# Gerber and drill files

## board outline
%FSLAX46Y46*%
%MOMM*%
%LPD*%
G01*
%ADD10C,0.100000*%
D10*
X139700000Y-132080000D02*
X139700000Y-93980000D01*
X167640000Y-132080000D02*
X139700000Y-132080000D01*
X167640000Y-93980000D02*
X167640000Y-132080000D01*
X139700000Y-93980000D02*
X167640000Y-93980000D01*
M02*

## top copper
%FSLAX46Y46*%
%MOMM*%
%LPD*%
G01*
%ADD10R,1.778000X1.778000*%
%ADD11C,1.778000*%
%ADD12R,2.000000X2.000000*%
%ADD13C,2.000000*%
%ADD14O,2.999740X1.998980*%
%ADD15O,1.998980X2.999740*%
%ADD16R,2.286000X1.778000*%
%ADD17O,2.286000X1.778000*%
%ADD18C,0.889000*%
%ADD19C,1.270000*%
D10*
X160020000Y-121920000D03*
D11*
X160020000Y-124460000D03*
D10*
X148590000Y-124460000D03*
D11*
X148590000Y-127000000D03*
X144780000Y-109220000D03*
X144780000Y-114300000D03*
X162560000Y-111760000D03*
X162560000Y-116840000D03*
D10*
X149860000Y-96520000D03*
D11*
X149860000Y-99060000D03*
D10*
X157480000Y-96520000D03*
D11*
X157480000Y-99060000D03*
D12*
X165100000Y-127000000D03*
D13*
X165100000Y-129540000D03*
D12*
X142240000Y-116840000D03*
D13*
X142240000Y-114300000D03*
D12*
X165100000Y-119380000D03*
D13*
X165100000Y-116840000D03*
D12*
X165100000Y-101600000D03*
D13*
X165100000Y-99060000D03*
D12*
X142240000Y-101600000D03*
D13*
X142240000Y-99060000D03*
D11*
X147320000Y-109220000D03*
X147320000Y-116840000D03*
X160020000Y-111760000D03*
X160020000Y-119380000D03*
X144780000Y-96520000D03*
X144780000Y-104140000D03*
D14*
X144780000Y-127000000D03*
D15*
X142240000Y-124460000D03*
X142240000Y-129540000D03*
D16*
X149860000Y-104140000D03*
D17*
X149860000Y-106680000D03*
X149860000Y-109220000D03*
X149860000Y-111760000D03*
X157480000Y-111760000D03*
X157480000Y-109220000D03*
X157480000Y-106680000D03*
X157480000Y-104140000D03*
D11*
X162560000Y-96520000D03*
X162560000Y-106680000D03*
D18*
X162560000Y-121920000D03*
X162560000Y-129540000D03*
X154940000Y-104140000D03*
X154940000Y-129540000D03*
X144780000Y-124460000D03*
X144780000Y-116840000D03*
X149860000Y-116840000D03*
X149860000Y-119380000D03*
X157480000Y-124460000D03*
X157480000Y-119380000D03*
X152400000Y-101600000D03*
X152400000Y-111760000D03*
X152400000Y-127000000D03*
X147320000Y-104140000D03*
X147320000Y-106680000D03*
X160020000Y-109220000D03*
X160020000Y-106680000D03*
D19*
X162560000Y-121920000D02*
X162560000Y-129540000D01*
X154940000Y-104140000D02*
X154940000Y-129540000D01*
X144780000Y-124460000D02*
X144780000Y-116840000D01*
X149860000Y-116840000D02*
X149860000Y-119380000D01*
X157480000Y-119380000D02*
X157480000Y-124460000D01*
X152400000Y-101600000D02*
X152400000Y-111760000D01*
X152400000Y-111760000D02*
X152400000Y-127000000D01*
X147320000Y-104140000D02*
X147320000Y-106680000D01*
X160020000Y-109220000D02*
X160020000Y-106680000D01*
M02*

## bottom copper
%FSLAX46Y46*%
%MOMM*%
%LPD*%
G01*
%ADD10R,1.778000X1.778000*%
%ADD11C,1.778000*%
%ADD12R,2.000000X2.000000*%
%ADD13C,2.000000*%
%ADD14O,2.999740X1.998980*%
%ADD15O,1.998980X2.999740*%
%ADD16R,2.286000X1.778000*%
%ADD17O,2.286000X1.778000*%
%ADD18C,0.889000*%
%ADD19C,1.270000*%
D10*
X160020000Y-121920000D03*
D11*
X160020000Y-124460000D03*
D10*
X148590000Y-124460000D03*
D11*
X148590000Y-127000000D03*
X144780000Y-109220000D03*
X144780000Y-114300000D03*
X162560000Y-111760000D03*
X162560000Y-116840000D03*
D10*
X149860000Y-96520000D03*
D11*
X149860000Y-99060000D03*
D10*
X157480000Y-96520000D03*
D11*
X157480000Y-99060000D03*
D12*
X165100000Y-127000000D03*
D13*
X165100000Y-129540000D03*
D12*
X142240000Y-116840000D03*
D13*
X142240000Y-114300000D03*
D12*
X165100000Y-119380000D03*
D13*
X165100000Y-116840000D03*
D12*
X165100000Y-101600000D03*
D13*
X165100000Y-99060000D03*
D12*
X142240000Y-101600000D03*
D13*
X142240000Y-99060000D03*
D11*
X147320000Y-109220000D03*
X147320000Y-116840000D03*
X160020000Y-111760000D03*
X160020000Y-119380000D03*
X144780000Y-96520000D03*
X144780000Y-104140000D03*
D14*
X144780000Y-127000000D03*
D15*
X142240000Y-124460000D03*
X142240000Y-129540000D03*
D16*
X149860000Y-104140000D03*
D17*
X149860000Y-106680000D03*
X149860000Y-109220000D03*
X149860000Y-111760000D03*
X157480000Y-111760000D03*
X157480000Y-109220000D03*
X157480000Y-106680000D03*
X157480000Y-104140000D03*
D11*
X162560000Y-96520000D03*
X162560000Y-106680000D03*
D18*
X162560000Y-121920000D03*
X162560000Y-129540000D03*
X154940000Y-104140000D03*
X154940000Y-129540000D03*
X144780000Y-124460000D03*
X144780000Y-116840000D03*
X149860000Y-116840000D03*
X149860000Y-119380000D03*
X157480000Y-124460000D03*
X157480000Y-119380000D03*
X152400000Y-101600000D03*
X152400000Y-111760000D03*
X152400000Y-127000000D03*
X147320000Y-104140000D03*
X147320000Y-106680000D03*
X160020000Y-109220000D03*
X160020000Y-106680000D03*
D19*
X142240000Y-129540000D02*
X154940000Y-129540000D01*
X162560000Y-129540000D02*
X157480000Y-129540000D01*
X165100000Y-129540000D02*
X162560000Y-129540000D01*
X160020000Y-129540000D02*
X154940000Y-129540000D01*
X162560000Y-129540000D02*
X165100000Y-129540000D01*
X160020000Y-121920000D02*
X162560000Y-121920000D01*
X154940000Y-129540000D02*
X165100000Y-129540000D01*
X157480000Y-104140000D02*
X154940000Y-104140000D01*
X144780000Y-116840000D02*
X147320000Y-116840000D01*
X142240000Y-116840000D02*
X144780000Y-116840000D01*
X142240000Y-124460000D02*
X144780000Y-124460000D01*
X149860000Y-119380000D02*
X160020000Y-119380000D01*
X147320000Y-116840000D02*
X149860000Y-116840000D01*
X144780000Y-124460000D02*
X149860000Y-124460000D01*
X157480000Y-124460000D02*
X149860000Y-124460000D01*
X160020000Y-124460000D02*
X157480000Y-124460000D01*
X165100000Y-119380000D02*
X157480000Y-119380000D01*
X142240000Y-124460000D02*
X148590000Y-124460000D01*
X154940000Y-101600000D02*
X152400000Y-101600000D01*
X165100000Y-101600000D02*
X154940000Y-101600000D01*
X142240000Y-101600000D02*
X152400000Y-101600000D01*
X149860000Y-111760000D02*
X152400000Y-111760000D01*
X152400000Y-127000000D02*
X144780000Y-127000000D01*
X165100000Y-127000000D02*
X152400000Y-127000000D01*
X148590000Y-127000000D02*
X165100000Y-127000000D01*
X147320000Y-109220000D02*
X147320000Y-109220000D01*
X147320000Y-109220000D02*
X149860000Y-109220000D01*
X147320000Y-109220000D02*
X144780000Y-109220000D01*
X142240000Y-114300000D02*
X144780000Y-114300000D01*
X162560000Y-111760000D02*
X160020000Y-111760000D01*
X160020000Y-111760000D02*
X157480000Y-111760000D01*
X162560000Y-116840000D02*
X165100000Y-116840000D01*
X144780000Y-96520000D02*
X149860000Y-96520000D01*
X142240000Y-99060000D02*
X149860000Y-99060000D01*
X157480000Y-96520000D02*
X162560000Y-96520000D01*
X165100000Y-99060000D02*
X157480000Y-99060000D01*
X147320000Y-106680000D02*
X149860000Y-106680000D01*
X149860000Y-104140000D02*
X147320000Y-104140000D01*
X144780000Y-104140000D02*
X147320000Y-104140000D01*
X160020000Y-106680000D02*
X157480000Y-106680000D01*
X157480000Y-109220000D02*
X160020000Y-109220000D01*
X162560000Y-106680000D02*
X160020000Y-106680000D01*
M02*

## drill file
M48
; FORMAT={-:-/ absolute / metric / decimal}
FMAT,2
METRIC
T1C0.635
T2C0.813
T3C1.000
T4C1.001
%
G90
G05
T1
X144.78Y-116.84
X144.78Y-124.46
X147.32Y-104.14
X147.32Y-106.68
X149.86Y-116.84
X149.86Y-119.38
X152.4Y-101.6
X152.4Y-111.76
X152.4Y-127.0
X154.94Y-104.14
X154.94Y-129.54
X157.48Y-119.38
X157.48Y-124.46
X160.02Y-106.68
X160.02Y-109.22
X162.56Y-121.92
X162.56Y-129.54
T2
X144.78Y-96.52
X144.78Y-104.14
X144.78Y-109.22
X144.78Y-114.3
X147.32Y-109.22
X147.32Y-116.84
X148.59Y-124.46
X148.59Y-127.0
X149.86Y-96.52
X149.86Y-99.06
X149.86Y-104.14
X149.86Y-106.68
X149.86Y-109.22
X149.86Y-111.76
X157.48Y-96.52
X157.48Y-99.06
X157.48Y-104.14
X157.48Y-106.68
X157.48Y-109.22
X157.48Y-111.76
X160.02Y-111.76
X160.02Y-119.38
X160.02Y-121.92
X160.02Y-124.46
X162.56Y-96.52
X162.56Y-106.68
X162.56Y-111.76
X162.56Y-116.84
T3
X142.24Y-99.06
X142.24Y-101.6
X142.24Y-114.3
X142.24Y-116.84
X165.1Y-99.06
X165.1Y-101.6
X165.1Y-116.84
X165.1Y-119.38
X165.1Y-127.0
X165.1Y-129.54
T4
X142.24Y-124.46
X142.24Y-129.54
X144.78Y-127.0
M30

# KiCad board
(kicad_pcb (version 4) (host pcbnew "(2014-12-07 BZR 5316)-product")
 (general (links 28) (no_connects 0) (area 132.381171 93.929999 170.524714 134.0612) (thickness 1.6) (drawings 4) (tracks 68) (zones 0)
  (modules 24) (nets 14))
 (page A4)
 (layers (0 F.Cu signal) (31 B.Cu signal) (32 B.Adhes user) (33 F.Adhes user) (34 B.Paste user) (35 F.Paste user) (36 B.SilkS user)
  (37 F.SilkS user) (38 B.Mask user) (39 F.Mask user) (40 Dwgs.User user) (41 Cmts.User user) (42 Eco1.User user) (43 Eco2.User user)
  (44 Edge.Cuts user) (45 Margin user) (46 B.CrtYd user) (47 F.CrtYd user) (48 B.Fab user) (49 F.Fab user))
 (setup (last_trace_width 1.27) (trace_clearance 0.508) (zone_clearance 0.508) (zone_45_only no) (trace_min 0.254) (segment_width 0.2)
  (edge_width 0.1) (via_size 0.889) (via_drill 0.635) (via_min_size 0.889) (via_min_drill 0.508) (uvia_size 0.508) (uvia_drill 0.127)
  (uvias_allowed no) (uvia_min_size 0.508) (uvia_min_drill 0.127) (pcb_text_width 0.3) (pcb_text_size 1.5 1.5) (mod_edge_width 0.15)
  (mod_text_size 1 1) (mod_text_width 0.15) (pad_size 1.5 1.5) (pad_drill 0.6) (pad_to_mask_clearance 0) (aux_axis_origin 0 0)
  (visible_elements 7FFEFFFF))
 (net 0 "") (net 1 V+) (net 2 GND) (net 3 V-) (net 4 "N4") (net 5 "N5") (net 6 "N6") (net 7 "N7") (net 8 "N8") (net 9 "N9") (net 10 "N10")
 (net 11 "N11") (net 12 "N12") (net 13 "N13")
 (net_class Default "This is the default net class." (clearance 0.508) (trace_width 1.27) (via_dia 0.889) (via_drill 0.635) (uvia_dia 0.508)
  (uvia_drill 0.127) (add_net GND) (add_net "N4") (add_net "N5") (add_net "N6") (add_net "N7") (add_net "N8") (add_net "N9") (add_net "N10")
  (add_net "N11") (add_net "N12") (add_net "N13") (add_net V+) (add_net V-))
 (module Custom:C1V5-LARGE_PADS (layer F.Cu) (at 160.02 123.19 270)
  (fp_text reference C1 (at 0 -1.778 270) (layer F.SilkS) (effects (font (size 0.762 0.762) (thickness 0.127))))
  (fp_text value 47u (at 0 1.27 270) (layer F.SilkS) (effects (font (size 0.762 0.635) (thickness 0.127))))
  (pad 1 thru_hole rect (at -1.27 0 270) (size 1.778 1.778) (drill 0.8128) (layers *.Cu *.Mask F.SilkS) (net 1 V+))
  (pad 2 thru_hole circle (at 1.27 0 270) (size 1.778 1.778) (drill 0.8128) (layers *.Cu *.Mask F.SilkS) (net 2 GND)))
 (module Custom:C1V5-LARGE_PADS (layer F.Cu) (at 148.59 125.73 270)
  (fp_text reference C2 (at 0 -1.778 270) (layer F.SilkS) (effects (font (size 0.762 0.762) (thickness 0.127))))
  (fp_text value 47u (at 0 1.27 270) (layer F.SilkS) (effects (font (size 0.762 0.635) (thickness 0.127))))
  (pad 1 thru_hole rect (at -1.27 0 270) (size 1.778 1.778) (drill 0.8128) (layers *.Cu *.Mask F.SilkS) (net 2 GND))
  (pad 2 thru_hole circle (at 1.27 0 270) (size 1.778 1.778) (drill 0.8128) (layers *.Cu *.Mask F.SilkS) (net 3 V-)))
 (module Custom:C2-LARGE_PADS (layer F.Cu) (at 144.78 111.76 270)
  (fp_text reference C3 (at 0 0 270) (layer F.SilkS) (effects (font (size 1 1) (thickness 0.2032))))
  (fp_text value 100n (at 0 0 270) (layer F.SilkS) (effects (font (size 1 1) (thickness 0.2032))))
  (pad 1 thru_hole circle (at -2.54 0 270) (size 1.778 1.778) (drill 0.8128) (layers *.Cu *.Mask F.SilkS) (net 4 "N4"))
  (pad 2 thru_hole circle (at 2.54 0 270) (size 1.778 1.778) (drill 0.8128) (layers *.Cu *.Mask F.SilkS) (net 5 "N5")))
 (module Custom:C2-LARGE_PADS (layer F.Cu) (at 162.56 114.3 270)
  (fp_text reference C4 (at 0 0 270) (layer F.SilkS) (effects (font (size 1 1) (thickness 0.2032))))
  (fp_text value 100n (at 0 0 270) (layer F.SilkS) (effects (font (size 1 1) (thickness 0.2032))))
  (pad 1 thru_hole circle (at -2.54 0 270) (size 1.778 1.778) (drill 0.8128) (layers *.Cu *.Mask F.SilkS) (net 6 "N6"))
  (pad 2 thru_hole circle (at 2.54 0 270) (size 1.778 1.778) (drill 0.8128) (layers *.Cu *.Mask F.SilkS) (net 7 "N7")))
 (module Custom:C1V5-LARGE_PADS (layer F.Cu) (at 149.86 97.79 270)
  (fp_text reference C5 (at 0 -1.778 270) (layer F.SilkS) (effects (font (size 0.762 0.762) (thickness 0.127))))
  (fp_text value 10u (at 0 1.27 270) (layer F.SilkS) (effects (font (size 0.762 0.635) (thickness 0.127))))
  (pad 1 thru_hole rect (at -1.27 0 270) (size 1.778 1.778) (drill 0.8128) (layers *.Cu *.Mask F.SilkS) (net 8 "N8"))
  (pad 2 thru_hole circle (at 1.27 0 270) (size 1.778 1.778) (drill 0.8128) (layers *.Cu *.Mask F.SilkS) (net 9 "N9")))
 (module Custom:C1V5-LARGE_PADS (layer F.Cu) (at 157.48 97.79 270)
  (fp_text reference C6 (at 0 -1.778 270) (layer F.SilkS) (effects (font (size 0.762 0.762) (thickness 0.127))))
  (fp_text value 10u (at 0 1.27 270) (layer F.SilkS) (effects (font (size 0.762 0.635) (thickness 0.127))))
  (pad 1 thru_hole rect (at -1.27 0 270) (size 1.778 1.778) (drill 0.8128) (layers *.Cu *.Mask F.SilkS) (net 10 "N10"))
  (pad 2 thru_hole circle (at 1.27 0 270) (size 1.778 1.778) (drill 0.8128) (layers *.Cu *.Mask F.SilkS) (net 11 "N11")))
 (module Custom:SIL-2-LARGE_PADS (layer F.Cu) (at 165.1 128.27 270)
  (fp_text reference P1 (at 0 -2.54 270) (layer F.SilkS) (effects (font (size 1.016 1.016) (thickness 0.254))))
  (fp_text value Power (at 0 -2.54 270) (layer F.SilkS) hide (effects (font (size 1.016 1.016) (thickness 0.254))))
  (pad 1 thru_hole rect (at -1.27 0 270) (size 2 2) (drill 1) (layers *.Cu *.Mask F.SilkS) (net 3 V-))
  (pad 2 thru_hole circle (at 1.27 0 270) (size 2 2) (drill 1) (layers *.Cu *.Mask F.SilkS) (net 1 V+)))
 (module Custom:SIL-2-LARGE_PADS (layer F.Cu) (at 142.24 115.57 90)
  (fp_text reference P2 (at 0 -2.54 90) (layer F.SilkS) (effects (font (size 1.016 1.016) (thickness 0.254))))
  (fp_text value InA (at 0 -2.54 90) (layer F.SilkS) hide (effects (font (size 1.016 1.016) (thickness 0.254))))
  (pad 1 thru_hole rect (at -1.27 0 90) (size 2 2) (drill 1) (layers *.Cu *.Mask F.SilkS) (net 2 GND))
  (pad 2 thru_hole circle (at 1.27 0 90) (size 2 2) (drill 1) (layers *.Cu *.Mask F.SilkS) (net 5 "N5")))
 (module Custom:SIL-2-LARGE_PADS (layer F.Cu) (at 165.1 118.11 90)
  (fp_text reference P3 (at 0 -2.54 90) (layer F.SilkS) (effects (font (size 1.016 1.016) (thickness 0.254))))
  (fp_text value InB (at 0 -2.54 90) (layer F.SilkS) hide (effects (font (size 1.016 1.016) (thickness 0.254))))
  (pad 1 thru_hole rect (at -1.27 0 90) (size 2 2) (drill 1) (layers *.Cu *.Mask F.SilkS) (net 2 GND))
  (pad 2 thru_hole circle (at 1.27 0 90) (size 2 2) (drill 1) (layers *.Cu *.Mask F.SilkS) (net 7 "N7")))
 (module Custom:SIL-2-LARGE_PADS (layer F.Cu) (at 165.1 100.33 90)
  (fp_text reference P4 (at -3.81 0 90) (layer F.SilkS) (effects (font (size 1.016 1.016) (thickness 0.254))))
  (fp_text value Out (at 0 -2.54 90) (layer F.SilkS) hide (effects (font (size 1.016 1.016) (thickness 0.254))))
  (pad 1 thru_hole rect (at -1.27 0 90) (size 2 2) (drill 1) (layers *.Cu *.Mask F.SilkS) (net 3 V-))
  (pad 2 thru_hole circle (at 1.27 0 90) (size 2 2) (drill 1) (layers *.Cu *.Mask F.SilkS) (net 11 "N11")))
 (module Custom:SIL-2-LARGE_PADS (layer F.Cu) (at 142.24 100.33 90)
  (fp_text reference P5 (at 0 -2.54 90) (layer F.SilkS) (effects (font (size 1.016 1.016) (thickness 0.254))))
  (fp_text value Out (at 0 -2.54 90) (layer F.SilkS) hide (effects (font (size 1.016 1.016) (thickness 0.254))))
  (pad 1 thru_hole rect (at -1.27 0 90) (size 2 2) (drill 1) (layers *.Cu *.Mask F.SilkS) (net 3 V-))
  (pad 2 thru_hole circle (at 1.27 0 90) (size 2 2) (drill 1) (layers *.Cu *.Mask F.SilkS) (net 9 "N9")))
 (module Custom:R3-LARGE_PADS (layer F.Cu) (at 147.32 113.03 270) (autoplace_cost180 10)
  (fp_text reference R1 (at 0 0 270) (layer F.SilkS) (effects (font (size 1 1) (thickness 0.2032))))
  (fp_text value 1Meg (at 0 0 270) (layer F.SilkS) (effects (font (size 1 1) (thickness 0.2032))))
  (pad 1 thru_hole circle (at -3.81 0 270) (size 1.778 1.778) (drill 0.8128) (layers *.Cu *.Mask F.SilkS) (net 4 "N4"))
  (pad 2 thru_hole circle (at 3.81 0 270) (size 1.778 1.778) (drill 0.8128) (layers *.Cu *.Mask F.SilkS) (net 2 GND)))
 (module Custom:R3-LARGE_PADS (layer F.Cu) (at 160.02 115.57 270) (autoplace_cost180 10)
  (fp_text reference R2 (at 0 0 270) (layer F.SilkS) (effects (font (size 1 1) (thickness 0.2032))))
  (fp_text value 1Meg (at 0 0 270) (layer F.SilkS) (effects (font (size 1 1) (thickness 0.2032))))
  (pad 1 thru_hole circle (at -3.81 0 270) (size 1.778 1.778) (drill 0.8128) (layers *.Cu *.Mask F.SilkS) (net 6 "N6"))
  (pad 2 thru_hole circle (at 3.81 0 270) (size 1.778 1.778) (drill 0.8128) (layers *.Cu *.Mask F.SilkS) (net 2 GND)))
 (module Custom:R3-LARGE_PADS (layer F.Cu) (at 144.78 100.33 270) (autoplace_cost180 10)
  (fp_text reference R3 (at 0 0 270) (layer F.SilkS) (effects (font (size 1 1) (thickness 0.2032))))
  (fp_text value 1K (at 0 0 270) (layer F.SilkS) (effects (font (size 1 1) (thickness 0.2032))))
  (pad 1 thru_hole circle (at -3.81 0 270) (size 1.778 1.778) (drill 0.8128) (layers *.Cu *.Mask F.SilkS) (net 8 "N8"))
  (pad 2 thru_hole circle (at 3.81 0 270) (size 1.778 1.778) (drill 0.8128) (layers *.Cu *.Mask F.SilkS) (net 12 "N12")))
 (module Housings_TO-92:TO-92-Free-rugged (layer F.Cu) (at 142.24 127)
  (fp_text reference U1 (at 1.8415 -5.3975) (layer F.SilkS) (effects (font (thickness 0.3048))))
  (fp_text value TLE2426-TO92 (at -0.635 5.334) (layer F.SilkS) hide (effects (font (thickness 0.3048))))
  (pad 2 thru_hole oval (at 2.54 0) (size 2.99974 1.99898) (drill 1.00076) (layers *.Cu *.Mask F.SilkS) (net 3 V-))
  (pad 1 thru_hole oval (at 0 -2.54) (size 1.99898 2.99974) (drill 1.00076) (layers *.Cu *.Mask F.SilkS) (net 2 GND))
  (pad 3 thru_hole oval (at 0 2.54) (size 1.99898 2.99974) (drill 1.00076) (layers *.Cu *.Mask F.SilkS) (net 1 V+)))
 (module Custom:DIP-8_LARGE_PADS (layer F.Cu) (at 153.67 107.95 270)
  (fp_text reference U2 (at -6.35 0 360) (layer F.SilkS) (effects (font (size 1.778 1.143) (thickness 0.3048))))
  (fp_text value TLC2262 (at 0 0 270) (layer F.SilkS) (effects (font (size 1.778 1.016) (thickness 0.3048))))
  (pad 1 thru_hole rect (at -3.81 3.81 270) (size 1.778 2.286) (drill 0.8128) (layers *.Cu *.Mask F.SilkS) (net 12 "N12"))
  (pad 2 thru_hole oval (at -1.27 3.81 270) (size 1.778 2.286) (drill 0.8128) (layers *.Cu *.Mask F.SilkS) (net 12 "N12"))
  (pad 3 thru_hole oval (at 1.27 3.81 270) (size 1.778 2.286) (drill 0.8128) (layers *.Cu *.Mask F.SilkS) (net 4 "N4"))
  (pad 4 thru_hole oval (at 3.81 3.81 270) (size 1.778 2.286) (drill 0.8128) (layers *.Cu *.Mask F.SilkS) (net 3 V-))
  (pad 5 thru_hole oval (at 3.81 -3.81 270) (size 1.778 2.286) (drill 0.8128) (layers *.Cu *.Mask F.SilkS) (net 6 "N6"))
  (pad 6 thru_hole oval (at 1.27 -3.81 270) (size 1.778 2.286) (drill 0.8128) (layers *.Cu *.Mask F.SilkS) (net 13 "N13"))
  (pad 7 thru_hole oval (at -1.27 -3.81 270) (size 1.778 2.286) (drill 0.8128) (layers *.Cu *.Mask F.SilkS) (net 13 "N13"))
  (pad 8 thru_hole oval (at -3.81 -3.81 270) (size 1.778 2.286) (drill 0.8128) (layers *.Cu *.Mask F.SilkS) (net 1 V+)))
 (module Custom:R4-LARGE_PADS (layer F.Cu) (at 162.56 101.6 270) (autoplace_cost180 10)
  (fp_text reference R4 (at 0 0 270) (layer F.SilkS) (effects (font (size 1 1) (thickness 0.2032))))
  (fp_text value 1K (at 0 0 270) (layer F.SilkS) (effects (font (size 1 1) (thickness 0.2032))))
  (pad 1 thru_hole circle (at -5.08 0 270) (size 1.778 1.778) (drill 0.8128) (layers *.Cu *.Mask F.SilkS) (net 10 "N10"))
  (pad 2 thru_hole circle (at 5.08 0 270) (size 1.778 1.778) (drill 0.8128) (layers *.Cu *.Mask F.SilkS) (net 13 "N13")))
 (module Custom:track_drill (layer F.Cu) (at 154.94 111.76)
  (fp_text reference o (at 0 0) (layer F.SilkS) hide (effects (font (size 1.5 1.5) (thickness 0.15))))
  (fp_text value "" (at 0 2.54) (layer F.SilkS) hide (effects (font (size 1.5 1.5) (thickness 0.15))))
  (pad 1 connect rect (at 0 0 45) (size 1.524 1.524) (layers B.SilkS B.Mask Dwgs.User) (die_length 0.254)))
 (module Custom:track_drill (layer F.Cu) (at 152.4 109.22)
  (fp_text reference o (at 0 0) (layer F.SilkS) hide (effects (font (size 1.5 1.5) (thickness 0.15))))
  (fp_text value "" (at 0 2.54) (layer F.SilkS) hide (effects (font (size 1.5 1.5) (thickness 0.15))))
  (pad 1 connect rect (at 0 0 45) (size 1.524 1.524) (layers *.Mask B.SilkS Dwgs.User) (die_length 0.254)))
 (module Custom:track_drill (layer F.Cu) (at 152.4 106.68)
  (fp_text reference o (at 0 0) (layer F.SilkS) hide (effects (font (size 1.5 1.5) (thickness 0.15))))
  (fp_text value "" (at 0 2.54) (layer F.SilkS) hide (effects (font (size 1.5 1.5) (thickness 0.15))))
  (pad 1 connect rect (at 0 0 45) (size 1.524 1.524) (layers *.Mask B.SilkS Dwgs.User) (die_length 0.254)))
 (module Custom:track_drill (layer F.Cu) (at 152.4 104.14)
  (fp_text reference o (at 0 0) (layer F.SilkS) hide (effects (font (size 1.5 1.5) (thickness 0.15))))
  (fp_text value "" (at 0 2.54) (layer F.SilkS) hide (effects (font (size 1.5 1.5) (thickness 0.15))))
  (pad 1 connect rect (at 0 0 45) (size 1.524 1.524) (layers *.Mask B.SilkS Dwgs.User) (die_length 0.254)))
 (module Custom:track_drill (layer F.Cu) (at 152.4 99.06)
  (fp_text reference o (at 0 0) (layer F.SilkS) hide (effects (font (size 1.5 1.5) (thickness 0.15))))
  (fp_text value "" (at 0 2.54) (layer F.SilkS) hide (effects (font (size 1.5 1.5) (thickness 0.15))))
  (pad 1 connect rect (at 0 0 45) (size 1.524 1.524) (layers *.Mask B.SilkS Dwgs.User) (die_length 0.254)))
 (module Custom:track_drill (layer F.Cu) (at 152.4 96.52)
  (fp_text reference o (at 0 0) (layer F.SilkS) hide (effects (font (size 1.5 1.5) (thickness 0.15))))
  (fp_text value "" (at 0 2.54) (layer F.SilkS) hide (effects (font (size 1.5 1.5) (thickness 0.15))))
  (pad 1 connect rect (at 0 0 45) (size 1.524 1.524) (layers *.Mask B.SilkS Dwgs.User) (die_length 0.254)))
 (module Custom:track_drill (layer F.Cu) (at 154.94 116.84)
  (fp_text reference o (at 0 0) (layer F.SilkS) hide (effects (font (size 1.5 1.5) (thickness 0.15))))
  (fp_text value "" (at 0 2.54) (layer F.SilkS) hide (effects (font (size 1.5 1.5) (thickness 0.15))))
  (pad 1 connect rect (at 0 0 45) (size 1.524 1.524) (layers *.Mask B.SilkS Dwgs.User) (die_length 0.254)))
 (gr_line (start 139.7 132.08) (end 139.7 93.98) (angle 90) (layer Edge.Cuts) (width 0.1))
 (gr_line (start 167.64 132.08) (end 139.7 132.08) (angle 90) (layer Edge.Cuts) (width 0.1))
 (gr_line (start 167.64 93.98) (end 167.64 132.08) (angle 90) (layer Edge.Cuts) (width 0.1))
 (gr_line (start 139.7 93.98) (end 167.64 93.98) (angle 90) (layer Edge.Cuts) (width 0.1))
 (segment (start 142.24 129.54) (end 154.94 129.54) (width 1.27) (layer B.Cu) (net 1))
 (segment (start 162.56 129.54) (end 157.48 129.54) (width 1.27) (layer B.Cu) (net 1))
 (segment (start 165.1 129.54) (end 162.56 129.54) (width 1.27) (layer B.Cu) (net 1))
 (segment (start 160.02 129.54) (end 154.94 129.54) (width 1.27) (layer B.Cu) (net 1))
 (segment (start 162.56 129.54) (end 165.1 129.54) (width 1.27) (layer B.Cu) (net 1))
 (via (at 162.56 121.92) (size 0.889) (layers F.Cu B.Cu) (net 1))
 (segment (start 162.56 121.92) (end 162.56 129.54) (width 1.27) (layer F.Cu) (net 1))
 (via (at 162.56 129.54) (size 0.889) (layers F.Cu B.Cu) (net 1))
 (segment (start 160.02 121.92) (end 162.56 121.92) (width 1.27) (layer B.Cu) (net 1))
 (segment (start 154.94 129.54) (end 165.1 129.54) (width 1.27) (layer B.Cu) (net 1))
 (via (at 154.94 104.14) (size 0.889) (layers F.Cu B.Cu) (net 1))
 (segment (start 154.94 104.14) (end 154.94 129.54) (width 1.27) (layer F.Cu) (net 1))
 (via (at 154.94 129.54) (size 0.889) (layers F.Cu B.Cu) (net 1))
 (segment (start 157.48 104.14) (end 154.94 104.14) (width 1.27) (layer B.Cu) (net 1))
 (segment (start 144.78 116.84) (end 147.32 116.84) (width 1.27) (layer B.Cu) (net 2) (status 10))
 (segment (start 142.24 116.84) (end 144.78 116.84) (width 1.27) (layer B.Cu) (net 2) (status 10))
 (via (at 144.78 124.46) (size 0.889) (layers F.Cu B.Cu) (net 2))
 (segment (start 144.78 124.46) (end 144.78 116.84) (width 1.27) (layer F.Cu) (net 2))
 (via (at 144.78 116.84) (size 0.889) (layers F.Cu B.Cu) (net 2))
 (segment (start 142.24 124.46) (end 144.78 124.46) (width 1.27) (layer B.Cu) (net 2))
 (via (at 149.86 116.84) (size 0.889) (layers F.Cu B.Cu) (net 2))
 (segment (start 149.86 116.84) (end 149.86 119.38) (width 1.27) (layer F.Cu) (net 2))
 (via (at 149.86 119.38) (size 0.889) (layers F.Cu B.Cu) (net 2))
 (segment (start 149.86 119.38) (end 160.02 119.38) (width 1.27) (layer B.Cu) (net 2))
 (segment (start 147.32 116.84) (end 149.86 116.84) (width 1.27) (layer B.Cu) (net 2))
 (segment (start 144.78 124.46) (end 149.86 124.46) (width 1.27) (layer B.Cu) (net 2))
 (segment (start 157.48 124.46) (end 149.86 124.46) (width 1.27) (layer B.Cu) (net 2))
 (segment (start 160.02 124.46) (end 157.48 124.46) (width 1.27) (layer B.Cu) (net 2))
 (segment (start 157.48 119.38) (end 157.48 124.46) (width 1.27) (layer F.Cu) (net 2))
 (via (at 157.48 124.46) (size 0.889) (layers F.Cu B.Cu) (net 2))
 (segment (start 165.1 119.38) (end 157.48 119.38) (width 1.27) (layer B.Cu) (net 2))
 (via (at 157.48 119.38) (size 0.889) (layers F.Cu B.Cu) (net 2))
 (segment (start 142.24 124.46) (end 148.59 124.46) (width 1.27) (layer B.Cu) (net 2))
 (segment (start 154.94 101.6) (end 152.4 101.6) (width 1.27) (layer B.Cu) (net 3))
 (segment (start 165.1 101.6) (end 154.94 101.6) (width 1.27) (layer B.Cu) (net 3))
 (segment (start 152.4 101.6) (end 152.4 111.76) (width 1.27) (layer F.Cu) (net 3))
 (via (at 152.4 101.6) (size 0.889) (layers F.Cu B.Cu) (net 3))
 (segment (start 142.24 101.6) (end 152.4 101.6) (width 1.27) (layer B.Cu) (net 3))
 (via (at 152.4 111.76) (size 0.889) (layers F.Cu B.Cu) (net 3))
 (segment (start 149.86 111.76) (end 152.4 111.76) (width 1.27) (layer B.Cu) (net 3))
 (segment (start 152.4 127) (end 144.78 127) (width 1.27) (layer B.Cu) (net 3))
 (segment (start 165.1 127) (end 152.4 127) (width 1.27) (layer B.Cu) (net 3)) (via (at 152.4 127) (size 0.889) (layers F.Cu B.Cu) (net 3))
 (segment (start 152.4 111.76) (end 152.4 127) (width 1.27) (layer F.Cu) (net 3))
 (segment (start 148.59 127) (end 165.1 127) (width 1.27) (layer B.Cu) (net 3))
 (segment (start 147.32 109.22) (end 147.32 109.22) (width 1.27) (layer B.Cu) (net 4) (status 30))
 (segment (start 147.32 109.22) (end 149.86 109.22) (width 1.27) (layer B.Cu) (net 4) (status 10))
 (segment (start 147.32 109.22) (end 144.78 109.22) (width 1.27) (layer B.Cu) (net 4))
 (segment (start 142.24 114.3) (end 144.78 114.3) (width 1.27) (layer B.Cu) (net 5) (status 10))
 (segment (start 162.56 111.76) (end 160.02 111.76) (width 1.27) (layer B.Cu) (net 6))
 (segment (start 160.02 111.76) (end 157.48 111.76) (width 1.27) (layer B.Cu) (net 6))
 (segment (start 162.56 116.84) (end 165.1 116.84) (width 1.27) (layer B.Cu) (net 7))
 (segment (start 144.78 96.52) (end 149.86 96.52) (width 1.27) (layer B.Cu) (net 8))
 (segment (start 142.24 99.06) (end 149.86 99.06) (width 1.27) (layer B.Cu) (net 9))
 (segment (start 157.48 96.52) (end 162.56 96.52) (width 1.27) (layer B.Cu) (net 10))
 (segment (start 165.1 99.06) (end 157.48 99.06) (width 1.27) (layer B.Cu) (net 11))
 (via (at 147.32 104.14) (size 0.889) (layers F.Cu B.Cu) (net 12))
 (segment (start 147.32 104.14) (end 147.32 106.68) (width 1.27) (layer F.Cu) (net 12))
 (via (at 147.32 106.68) (size 0.889) (layers F.Cu B.Cu) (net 12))
 (segment (start 147.32 106.68) (end 149.86 106.68) (width 1.27) (layer B.Cu) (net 12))
 (segment (start 149.86 104.14) (end 147.32 104.14) (width 1.27) (layer B.Cu) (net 12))
 (segment (start 144.78 104.14) (end 147.32 104.14) (width 1.27) (layer B.Cu) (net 12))
 (via (at 160.02 109.22) (size 0.889) (layers F.Cu B.Cu) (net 13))
 (segment (start 160.02 109.22) (end 160.02 106.68) (width 1.27) (layer F.Cu) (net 13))
 (via (at 160.02 106.68) (size 0.889) (layers F.Cu B.Cu) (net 13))
 (segment (start 160.02 106.68) (end 157.48 106.68) (width 1.27) (layer B.Cu) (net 13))
 (segment (start 157.48 109.22) (end 160.02 109.22) (width 1.27) (layer B.Cu) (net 13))
 (segment (start 162.56 106.68) (end 160.02 106.68) (width 1.27) (layer B.Cu) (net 13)))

